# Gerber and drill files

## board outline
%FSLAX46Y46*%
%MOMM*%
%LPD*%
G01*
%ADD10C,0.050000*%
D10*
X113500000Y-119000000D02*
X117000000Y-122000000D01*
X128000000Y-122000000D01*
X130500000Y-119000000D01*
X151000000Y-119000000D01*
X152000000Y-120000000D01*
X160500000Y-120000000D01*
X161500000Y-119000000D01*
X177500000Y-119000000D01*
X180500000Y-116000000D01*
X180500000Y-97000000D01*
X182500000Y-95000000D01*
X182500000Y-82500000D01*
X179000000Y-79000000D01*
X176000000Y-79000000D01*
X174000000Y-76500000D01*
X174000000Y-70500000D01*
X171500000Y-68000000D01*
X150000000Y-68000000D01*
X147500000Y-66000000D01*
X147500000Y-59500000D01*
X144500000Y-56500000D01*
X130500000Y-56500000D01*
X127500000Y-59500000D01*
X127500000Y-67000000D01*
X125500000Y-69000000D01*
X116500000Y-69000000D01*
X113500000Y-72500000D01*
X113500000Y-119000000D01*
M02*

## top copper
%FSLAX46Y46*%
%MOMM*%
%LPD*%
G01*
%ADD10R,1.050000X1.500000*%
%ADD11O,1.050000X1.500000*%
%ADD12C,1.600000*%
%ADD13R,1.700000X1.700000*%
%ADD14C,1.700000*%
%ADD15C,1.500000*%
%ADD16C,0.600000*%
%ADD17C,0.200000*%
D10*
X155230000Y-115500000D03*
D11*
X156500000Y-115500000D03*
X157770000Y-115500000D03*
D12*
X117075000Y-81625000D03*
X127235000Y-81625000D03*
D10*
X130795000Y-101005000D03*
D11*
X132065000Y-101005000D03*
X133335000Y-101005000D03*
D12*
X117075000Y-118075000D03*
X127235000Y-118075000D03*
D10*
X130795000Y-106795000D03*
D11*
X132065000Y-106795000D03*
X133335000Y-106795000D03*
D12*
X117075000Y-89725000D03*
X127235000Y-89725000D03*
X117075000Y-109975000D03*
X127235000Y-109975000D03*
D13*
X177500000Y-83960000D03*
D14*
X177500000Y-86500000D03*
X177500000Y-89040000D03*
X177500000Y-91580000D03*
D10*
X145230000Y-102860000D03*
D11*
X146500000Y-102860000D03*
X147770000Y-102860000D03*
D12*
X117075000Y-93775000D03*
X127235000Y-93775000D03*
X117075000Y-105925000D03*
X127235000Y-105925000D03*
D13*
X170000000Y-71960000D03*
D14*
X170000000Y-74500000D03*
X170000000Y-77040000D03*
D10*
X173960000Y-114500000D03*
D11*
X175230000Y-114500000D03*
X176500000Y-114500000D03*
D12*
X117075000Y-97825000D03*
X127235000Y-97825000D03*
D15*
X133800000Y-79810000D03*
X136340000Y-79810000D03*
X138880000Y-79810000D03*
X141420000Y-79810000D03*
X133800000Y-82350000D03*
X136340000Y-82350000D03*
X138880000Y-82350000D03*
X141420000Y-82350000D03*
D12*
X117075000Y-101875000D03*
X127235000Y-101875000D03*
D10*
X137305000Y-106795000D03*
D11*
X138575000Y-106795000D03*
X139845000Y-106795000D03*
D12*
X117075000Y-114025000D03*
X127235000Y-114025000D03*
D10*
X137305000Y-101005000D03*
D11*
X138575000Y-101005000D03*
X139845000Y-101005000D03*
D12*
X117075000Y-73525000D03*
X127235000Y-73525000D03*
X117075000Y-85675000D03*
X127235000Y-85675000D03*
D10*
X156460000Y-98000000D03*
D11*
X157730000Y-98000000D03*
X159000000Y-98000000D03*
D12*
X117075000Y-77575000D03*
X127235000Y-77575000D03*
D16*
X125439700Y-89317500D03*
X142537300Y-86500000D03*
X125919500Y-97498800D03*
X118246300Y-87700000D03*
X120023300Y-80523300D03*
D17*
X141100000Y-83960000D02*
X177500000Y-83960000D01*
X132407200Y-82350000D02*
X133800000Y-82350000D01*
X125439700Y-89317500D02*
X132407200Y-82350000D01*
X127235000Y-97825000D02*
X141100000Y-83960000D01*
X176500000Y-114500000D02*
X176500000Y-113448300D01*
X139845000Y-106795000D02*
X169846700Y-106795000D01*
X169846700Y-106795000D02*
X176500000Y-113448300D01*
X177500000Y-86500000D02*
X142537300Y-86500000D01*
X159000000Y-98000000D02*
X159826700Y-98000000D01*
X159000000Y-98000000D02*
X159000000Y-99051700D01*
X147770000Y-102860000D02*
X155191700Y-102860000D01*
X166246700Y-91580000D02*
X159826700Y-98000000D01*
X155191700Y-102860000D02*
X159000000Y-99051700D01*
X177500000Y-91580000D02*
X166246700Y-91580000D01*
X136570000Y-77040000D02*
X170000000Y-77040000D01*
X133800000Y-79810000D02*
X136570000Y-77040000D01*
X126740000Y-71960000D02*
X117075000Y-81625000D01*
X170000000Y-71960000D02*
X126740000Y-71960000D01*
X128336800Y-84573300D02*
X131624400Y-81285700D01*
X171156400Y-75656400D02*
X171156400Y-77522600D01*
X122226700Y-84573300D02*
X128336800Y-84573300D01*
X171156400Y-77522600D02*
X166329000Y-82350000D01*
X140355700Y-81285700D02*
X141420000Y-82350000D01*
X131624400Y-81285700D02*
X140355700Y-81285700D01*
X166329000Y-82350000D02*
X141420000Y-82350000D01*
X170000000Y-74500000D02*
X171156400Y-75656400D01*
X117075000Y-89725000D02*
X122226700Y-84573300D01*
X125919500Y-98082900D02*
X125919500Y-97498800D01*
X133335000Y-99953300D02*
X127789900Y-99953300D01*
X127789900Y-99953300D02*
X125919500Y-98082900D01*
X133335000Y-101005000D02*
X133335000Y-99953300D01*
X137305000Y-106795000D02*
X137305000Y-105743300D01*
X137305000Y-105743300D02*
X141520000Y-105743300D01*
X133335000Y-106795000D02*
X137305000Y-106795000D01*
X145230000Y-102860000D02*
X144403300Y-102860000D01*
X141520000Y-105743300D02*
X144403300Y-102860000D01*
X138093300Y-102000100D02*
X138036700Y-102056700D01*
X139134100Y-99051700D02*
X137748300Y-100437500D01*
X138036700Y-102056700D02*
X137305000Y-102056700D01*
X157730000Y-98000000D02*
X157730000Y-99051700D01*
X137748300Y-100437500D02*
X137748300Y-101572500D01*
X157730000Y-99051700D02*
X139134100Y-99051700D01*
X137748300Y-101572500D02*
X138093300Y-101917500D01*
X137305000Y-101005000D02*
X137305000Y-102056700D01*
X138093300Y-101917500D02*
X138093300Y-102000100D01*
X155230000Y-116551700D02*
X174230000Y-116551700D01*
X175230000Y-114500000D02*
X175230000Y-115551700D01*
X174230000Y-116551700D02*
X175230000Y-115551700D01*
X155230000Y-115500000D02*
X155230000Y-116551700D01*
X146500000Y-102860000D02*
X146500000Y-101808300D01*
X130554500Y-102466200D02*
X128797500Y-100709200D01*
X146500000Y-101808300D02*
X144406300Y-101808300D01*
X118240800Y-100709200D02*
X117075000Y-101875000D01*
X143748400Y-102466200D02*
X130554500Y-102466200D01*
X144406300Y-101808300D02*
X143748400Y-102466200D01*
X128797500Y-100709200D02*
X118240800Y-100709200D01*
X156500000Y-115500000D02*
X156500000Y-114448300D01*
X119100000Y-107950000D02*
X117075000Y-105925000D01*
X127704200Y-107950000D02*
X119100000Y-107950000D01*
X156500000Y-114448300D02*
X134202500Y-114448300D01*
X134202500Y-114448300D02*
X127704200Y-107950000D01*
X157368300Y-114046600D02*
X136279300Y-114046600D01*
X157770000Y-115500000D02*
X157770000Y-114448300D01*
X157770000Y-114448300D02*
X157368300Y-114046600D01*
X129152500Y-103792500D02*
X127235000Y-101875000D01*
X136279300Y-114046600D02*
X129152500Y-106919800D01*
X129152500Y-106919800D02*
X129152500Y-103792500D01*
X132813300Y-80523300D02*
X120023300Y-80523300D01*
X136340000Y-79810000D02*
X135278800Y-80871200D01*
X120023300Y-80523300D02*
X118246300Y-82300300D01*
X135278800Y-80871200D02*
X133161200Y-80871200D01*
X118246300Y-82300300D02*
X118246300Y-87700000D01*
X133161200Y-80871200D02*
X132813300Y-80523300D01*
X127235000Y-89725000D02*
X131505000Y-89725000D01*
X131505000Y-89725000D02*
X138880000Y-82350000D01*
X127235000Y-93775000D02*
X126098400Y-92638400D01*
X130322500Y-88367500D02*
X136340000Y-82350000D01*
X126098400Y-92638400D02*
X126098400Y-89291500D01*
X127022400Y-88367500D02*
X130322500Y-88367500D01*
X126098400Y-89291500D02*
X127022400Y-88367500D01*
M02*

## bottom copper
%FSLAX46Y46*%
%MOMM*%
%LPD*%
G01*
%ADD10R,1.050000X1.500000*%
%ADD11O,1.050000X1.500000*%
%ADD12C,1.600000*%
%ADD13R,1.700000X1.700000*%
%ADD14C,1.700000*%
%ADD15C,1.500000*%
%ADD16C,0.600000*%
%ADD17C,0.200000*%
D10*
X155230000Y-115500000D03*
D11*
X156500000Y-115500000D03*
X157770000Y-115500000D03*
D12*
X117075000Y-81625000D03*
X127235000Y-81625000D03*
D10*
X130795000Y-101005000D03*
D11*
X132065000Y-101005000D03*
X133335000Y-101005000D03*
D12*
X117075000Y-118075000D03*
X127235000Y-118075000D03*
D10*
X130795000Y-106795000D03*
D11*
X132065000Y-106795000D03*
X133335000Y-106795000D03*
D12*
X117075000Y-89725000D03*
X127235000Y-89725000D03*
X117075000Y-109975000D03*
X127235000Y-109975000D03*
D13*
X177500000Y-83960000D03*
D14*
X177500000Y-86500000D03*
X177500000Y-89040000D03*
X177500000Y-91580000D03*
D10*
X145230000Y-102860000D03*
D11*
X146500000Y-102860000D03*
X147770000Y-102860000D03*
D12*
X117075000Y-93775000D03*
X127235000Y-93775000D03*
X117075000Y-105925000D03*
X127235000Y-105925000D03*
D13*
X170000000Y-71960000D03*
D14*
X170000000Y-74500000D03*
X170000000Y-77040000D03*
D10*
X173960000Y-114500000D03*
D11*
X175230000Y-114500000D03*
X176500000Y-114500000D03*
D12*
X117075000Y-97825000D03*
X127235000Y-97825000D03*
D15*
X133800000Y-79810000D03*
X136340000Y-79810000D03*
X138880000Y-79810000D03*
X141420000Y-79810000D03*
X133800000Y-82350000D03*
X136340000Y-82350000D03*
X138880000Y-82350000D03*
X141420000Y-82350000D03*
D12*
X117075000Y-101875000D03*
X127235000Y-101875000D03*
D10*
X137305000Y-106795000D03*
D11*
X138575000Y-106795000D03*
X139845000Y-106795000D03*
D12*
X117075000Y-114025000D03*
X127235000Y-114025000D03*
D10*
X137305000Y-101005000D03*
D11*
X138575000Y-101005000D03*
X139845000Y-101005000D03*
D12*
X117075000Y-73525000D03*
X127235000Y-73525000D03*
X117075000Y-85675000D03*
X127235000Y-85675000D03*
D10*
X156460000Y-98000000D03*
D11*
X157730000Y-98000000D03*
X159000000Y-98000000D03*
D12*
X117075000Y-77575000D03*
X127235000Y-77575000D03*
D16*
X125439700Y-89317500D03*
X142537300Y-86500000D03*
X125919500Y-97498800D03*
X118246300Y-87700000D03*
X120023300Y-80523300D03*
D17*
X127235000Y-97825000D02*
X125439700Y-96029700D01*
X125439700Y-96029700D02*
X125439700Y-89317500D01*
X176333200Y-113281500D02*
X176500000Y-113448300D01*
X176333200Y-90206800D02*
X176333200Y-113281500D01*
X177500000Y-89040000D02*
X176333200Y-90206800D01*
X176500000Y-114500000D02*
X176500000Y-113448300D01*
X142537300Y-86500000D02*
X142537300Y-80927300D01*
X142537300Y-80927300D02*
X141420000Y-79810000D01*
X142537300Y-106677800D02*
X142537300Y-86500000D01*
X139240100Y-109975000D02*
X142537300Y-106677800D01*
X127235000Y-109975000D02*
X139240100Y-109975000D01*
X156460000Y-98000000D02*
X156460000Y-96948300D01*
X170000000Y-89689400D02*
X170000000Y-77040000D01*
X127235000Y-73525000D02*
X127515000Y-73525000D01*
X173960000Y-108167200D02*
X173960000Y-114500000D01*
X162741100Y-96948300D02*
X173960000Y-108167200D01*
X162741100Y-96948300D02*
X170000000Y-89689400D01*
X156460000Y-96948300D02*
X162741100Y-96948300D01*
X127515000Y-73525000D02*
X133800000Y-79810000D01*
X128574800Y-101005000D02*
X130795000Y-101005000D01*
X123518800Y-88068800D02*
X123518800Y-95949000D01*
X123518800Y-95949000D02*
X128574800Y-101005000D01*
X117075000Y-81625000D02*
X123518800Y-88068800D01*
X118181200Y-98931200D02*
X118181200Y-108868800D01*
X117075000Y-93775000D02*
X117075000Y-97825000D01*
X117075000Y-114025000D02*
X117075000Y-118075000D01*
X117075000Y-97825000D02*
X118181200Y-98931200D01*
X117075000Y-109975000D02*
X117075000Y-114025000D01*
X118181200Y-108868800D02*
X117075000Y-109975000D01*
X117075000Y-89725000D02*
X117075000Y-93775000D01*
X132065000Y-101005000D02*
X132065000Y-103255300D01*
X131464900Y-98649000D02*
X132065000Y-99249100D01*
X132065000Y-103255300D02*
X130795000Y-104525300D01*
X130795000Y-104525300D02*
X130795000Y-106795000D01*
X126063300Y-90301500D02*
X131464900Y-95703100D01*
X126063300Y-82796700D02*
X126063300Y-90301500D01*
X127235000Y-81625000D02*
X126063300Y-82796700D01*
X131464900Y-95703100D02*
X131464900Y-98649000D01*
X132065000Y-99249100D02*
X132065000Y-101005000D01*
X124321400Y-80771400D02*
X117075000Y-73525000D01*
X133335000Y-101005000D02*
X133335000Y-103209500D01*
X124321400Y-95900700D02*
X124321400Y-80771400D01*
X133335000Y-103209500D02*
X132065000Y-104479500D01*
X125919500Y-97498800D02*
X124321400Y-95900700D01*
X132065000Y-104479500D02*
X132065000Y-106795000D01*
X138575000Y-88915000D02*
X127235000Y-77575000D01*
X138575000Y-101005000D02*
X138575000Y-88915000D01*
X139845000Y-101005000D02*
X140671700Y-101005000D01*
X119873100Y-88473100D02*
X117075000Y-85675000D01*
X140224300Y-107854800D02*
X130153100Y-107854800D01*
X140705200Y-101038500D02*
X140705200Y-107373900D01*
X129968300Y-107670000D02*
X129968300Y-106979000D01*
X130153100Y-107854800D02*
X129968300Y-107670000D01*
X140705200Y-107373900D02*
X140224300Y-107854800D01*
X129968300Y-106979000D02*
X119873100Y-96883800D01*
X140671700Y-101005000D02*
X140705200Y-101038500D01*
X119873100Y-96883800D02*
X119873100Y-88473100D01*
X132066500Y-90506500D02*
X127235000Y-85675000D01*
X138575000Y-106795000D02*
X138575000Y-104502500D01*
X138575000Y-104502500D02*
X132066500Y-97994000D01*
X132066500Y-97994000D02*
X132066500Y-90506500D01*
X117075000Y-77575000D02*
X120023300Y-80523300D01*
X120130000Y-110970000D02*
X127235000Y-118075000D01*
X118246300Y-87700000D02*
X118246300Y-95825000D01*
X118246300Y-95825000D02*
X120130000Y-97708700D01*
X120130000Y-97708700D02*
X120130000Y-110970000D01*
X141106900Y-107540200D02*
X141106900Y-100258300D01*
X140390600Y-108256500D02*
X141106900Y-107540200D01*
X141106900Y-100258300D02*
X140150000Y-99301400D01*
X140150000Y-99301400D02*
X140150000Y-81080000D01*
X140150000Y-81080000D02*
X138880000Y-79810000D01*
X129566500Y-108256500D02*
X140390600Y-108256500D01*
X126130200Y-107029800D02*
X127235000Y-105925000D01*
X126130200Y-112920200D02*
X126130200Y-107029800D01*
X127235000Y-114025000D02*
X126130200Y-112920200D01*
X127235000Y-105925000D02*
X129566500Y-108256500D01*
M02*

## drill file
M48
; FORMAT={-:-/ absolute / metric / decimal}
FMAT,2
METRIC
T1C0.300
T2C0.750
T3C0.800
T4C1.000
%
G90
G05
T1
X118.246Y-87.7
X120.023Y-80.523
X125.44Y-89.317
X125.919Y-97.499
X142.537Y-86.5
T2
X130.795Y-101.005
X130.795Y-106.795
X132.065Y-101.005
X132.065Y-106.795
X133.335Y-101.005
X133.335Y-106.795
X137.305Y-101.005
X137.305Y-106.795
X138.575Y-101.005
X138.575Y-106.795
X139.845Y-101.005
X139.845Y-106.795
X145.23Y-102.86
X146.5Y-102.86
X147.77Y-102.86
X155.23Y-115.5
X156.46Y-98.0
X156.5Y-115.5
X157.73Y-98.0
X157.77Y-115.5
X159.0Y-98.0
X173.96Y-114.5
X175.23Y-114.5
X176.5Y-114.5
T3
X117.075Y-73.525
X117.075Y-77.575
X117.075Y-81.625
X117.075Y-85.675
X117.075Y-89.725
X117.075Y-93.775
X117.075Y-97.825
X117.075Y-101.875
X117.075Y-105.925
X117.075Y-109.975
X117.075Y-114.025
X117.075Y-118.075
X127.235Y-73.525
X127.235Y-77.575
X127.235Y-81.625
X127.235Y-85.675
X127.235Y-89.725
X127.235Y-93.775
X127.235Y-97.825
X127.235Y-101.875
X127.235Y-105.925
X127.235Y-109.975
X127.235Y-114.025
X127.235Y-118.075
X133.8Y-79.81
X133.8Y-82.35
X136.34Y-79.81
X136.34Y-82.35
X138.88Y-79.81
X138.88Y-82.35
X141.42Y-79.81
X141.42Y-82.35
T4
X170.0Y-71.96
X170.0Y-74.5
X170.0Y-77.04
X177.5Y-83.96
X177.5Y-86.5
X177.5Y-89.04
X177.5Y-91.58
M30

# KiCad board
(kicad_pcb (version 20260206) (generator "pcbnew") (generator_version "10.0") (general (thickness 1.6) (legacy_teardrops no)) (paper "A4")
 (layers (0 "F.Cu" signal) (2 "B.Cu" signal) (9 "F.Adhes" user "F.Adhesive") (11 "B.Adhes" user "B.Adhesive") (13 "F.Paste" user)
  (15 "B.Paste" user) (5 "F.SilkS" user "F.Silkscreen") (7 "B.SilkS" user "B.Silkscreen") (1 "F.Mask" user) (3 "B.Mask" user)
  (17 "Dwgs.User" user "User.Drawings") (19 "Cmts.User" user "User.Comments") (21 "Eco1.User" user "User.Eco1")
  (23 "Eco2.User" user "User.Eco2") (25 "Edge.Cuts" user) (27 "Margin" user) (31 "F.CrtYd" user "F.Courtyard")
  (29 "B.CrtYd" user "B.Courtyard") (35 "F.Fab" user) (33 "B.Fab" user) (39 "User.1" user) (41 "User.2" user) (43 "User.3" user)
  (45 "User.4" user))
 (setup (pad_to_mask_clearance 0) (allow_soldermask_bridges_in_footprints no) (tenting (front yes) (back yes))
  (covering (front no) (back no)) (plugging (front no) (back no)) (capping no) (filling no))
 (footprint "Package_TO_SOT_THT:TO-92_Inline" (layer "F.Cu") (at 155.23 115.5)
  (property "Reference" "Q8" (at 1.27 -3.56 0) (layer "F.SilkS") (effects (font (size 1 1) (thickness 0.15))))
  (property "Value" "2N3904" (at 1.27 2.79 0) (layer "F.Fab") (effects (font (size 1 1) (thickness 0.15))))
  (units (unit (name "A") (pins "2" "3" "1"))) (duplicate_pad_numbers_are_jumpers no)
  (pad "1" thru_hole rect (at 0 0) (size 1.05 1.5) (drill 0.75) (layers "*.Cu" "*.Mask") (remove_unused_layers no) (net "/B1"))
  (pad "2" thru_hole oval (at 1.27 0) (size 1.05 1.5) (drill 0.75) (layers "*.Cu" "*.Mask") (remove_unused_layers no) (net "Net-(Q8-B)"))
  (pad "3" thru_hole oval (at 2.54 0) (size 1.05 1.5) (drill 0.75) (layers "*.Cu" "*.Mask") (remove_unused_layers no) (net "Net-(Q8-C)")))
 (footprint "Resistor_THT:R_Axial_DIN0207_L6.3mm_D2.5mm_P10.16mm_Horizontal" (layer "F.Cu") (at 117.075 81.625)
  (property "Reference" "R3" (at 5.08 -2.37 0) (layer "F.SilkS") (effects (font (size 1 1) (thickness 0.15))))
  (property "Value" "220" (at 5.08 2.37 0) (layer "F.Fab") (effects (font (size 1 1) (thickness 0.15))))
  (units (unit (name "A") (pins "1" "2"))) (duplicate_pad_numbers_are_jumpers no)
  (pad "1" thru_hole circle (at 0 0) (size 1.6 1.6) (drill 0.8) (layers "*.Cu" "*.Mask") (remove_unused_layers no) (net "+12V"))
  (pad "2" thru_hole circle (at 10.16 0) (size 1.6 1.6) (drill 0.8) (layers "*.Cu" "*.Mask") (remove_unused_layers no) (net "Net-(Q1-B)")))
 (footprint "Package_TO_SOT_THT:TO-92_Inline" (layer "F.Cu") (at 130.795 101.005)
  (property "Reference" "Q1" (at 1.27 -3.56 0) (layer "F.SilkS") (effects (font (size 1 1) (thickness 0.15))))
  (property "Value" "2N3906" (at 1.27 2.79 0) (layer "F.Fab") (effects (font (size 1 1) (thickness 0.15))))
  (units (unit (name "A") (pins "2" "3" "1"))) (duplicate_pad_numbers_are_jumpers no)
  (pad "1" thru_hole rect (at 0 0) (size 1.05 1.5) (drill 0.75) (layers "*.Cu" "*.Mask") (remove_unused_layers no) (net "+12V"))
  (pad "2" thru_hole oval (at 1.27 0) (size 1.05 1.5) (drill 0.75) (layers "*.Cu" "*.Mask") (remove_unused_layers no) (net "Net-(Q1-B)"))
  (pad "3" thru_hole oval (at 2.54 0) (size 1.05 1.5) (drill 0.75) (layers "*.Cu" "*.Mask") (remove_unused_layers no) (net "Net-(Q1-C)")))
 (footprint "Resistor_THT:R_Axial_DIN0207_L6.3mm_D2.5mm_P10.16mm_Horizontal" (layer "F.Cu") (at 117.075 118.075)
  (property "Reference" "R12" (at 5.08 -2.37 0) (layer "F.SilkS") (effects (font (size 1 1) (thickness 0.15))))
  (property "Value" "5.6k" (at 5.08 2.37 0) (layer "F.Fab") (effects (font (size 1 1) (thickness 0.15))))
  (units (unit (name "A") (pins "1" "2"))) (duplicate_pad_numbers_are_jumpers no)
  (pad "1" thru_hole circle (at 0 0) (size 1.6 1.6) (drill 0.8) (layers "*.Cu" "*.Mask") (remove_unused_layers no) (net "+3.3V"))
  (pad "2" thru_hole circle (at 10.16 0) (size 1.6 1.6) (drill 0.8) (layers "*.Cu" "*.Mask") (remove_unused_layers no) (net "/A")))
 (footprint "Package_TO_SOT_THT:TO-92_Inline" (layer "F.Cu") (at 130.795 106.795)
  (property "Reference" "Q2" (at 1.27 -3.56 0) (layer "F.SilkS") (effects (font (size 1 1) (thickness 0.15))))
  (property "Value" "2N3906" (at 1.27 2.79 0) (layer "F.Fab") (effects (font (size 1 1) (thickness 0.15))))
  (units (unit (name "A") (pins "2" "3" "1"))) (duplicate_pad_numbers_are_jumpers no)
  (pad "1" thru_hole rect (at 0 0) (size 1.05 1.5) (drill 0.75) (layers "*.Cu" "*.Mask") (remove_unused_layers no) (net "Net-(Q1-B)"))
  (pad "2" thru_hole oval (at 1.27 0) (size 1.05 1.5) (drill 0.75) (layers "*.Cu" "*.Mask") (remove_unused_layers no) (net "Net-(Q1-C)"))
  (pad "3" thru_hole oval (at 2.54 0) (size 1.05 1.5) (drill 0.75) (layers "*.Cu" "*.Mask") (remove_unused_layers no) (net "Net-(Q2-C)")))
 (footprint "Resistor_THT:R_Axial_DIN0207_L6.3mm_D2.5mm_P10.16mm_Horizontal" (layer "F.Cu") (at 117.075 89.725)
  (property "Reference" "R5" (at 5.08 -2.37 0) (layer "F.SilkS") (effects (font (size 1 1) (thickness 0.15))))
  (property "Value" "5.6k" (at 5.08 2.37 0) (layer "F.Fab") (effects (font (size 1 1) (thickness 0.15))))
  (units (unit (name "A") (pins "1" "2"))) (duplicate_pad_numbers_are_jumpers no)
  (pad "1" thru_hole circle (at 0 0) (size 1.6 1.6) (drill 0.8) (layers "*.Cu" "*.Mask") (remove_unused_layers no) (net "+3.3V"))
  (pad "2" thru_hole circle (at 10.16 0) (size 1.6 1.6) (drill 0.8) (layers "*.Cu" "*.Mask") (remove_unused_layers no)
   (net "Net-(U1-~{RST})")))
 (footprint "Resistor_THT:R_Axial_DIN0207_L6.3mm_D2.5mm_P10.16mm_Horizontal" (layer "F.Cu") (at 117.075 109.975)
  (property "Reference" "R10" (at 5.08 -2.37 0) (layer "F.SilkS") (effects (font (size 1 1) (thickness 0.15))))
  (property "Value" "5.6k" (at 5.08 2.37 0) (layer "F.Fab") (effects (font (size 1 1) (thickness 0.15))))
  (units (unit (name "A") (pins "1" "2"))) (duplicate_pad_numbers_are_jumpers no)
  (pad "1" thru_hole circle (at 0 0) (size 1.6 1.6) (drill 0.8) (layers "*.Cu" "*.Mask") (remove_unused_layers no) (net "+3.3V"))
  (pad "2" thru_hole circle (at 10.16 0) (size 1.6 1.6) (drill 0.8) (layers "*.Cu" "*.Mask") (remove_unused_layers no) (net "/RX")))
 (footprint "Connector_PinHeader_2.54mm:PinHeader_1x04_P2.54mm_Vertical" (layer "F.Cu") (at 177.5 83.96)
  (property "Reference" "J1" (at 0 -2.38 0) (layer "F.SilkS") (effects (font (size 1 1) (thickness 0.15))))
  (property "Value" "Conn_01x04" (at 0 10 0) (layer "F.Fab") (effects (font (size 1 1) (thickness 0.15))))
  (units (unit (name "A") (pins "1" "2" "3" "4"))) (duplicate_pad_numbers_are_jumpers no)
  (pad "1" thru_hole rect (at 0 0) (size 1.7 1.7) (drill 1) (layers "*.Cu" "*.Mask") (remove_unused_layers no) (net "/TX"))
  (pad "2" thru_hole circle (at 0 2.54) (size 1.7 1.7) (drill 1) (layers "*.Cu" "*.Mask") (remove_unused_layers no) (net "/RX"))
  (pad "3" thru_hole circle (at 0 5.08) (size 1.7 1.7) (drill 1) (layers "*.Cu" "*.Mask") (remove_unused_layers no) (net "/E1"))
  (pad "4" thru_hole circle (at 0 7.62) (size 1.7 1.7) (drill 1) (layers "*.Cu" "*.Mask") (remove_unused_layers no) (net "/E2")))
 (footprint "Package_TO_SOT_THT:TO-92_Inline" (layer "F.Cu") (at 145.23 102.86)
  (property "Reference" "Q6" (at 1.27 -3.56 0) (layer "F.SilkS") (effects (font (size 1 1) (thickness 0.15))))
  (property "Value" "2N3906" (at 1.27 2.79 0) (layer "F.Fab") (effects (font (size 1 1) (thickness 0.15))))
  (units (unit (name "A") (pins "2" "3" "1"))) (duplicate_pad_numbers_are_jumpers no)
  (pad "1" thru_hole rect (at 0 0) (size 1.05 1.5) (drill 0.75) (layers "*.Cu" "*.Mask") (remove_unused_layers no) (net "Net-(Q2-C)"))
  (pad "2" thru_hole oval (at 1.27 0) (size 1.05 1.5) (drill 0.75) (layers "*.Cu" "*.Mask") (remove_unused_layers no) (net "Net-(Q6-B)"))
  (pad "3" thru_hole oval (at 2.54 0) (size 1.05 1.5) (drill 0.75) (layers "*.Cu" "*.Mask") (remove_unused_layers no) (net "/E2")))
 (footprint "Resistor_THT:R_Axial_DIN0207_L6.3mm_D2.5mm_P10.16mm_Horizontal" (layer "F.Cu") (at 117.075 93.775)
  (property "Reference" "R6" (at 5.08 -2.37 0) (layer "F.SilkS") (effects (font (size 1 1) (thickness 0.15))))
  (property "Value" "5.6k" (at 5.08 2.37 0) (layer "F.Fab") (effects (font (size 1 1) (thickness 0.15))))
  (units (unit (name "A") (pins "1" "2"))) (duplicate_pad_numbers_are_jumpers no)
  (pad "1" thru_hole circle (at 0 0) (size 1.6 1.6) (drill 0.8) (layers "*.Cu" "*.Mask") (remove_unused_layers no) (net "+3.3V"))
  (pad "2" thru_hole circle (at 10.16 0) (size 1.6 1.6) (drill 0.8) (layers "*.Cu" "*.Mask") (remove_unused_layers no) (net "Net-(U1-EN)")))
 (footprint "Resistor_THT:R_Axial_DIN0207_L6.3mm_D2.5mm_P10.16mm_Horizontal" (layer "F.Cu") (at 117.075 105.925)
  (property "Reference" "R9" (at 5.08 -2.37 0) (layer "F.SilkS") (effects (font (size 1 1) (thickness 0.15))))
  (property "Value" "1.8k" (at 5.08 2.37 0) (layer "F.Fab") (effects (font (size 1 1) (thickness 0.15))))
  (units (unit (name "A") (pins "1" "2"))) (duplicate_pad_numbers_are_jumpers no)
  (pad "1" thru_hole circle (at 0 0) (size 1.6 1.6) (drill 0.8) (layers "*.Cu" "*.Mask") (remove_unused_layers no) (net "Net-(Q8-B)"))
  (pad "2" thru_hole circle (at 10.16 0) (size 1.6 1.6) (drill 0.8) (layers "*.Cu" "*.Mask") (remove_unused_layers no) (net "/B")))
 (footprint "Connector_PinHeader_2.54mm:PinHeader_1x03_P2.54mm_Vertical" (layer "F.Cu") (at 170 71.96)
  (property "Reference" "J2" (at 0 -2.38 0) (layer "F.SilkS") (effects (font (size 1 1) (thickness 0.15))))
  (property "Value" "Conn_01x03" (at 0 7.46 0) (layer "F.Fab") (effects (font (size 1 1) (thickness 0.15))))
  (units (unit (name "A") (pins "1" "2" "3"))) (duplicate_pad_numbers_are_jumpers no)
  (pad "1" thru_hole rect (at 0 0) (size 1.7 1.7) (drill 1) (layers "*.Cu" "*.Mask") (remove_unused_layers no) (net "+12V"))
  (pad "2" thru_hole circle (at 0 2.54) (size 1.7 1.7) (drill 1) (layers "*.Cu" "*.Mask") (remove_unused_layers no) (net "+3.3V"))
  (pad "3" thru_hole circle (at 0 5.08) (size 1.7 1.7) (drill 1) (layers "*.Cu" "*.Mask") (remove_unused_layers no) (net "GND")))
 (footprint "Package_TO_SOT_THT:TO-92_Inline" (layer "F.Cu") (at 173.96 114.5)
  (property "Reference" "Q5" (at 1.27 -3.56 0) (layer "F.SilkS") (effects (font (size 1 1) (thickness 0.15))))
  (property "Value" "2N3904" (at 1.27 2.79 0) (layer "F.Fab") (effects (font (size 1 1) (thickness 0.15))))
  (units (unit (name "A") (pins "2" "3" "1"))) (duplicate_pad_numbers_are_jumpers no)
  (pad "1" thru_hole rect (at 0 0) (size 1.05 1.5) (drill 0.75) (layers "*.Cu" "*.Mask") (remove_unused_layers no) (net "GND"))
  (pad "2" thru_hole oval (at 1.27 0) (size 1.05 1.5) (drill 0.75) (layers "*.Cu" "*.Mask") (remove_unused_layers no) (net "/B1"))
  (pad "3" thru_hole oval (at 2.54 0) (size 1.05 1.5) (drill 0.75) (layers "*.Cu" "*.Mask") (remove_unused_layers no) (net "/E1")))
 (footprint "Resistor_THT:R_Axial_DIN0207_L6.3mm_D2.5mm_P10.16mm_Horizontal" (layer "F.Cu") (at 117.075 97.825)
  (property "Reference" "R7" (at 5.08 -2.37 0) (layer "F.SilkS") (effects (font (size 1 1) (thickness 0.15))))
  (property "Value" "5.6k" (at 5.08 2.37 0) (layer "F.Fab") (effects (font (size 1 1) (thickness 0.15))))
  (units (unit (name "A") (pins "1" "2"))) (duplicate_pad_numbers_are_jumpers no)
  (pad "1" thru_hole circle (at 0 0) (size 1.6 1.6) (drill 0.8) (layers "*.Cu" "*.Mask") (remove_unused_layers no) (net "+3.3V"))
  (pad "2" thru_hole circle (at 10.16 0) (size 1.6 1.6) (drill 0.8) (layers "*.Cu" "*.Mask") (remove_unused_layers no) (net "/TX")))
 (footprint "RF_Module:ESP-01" (layer "F.Cu") (at 133.8 79.81)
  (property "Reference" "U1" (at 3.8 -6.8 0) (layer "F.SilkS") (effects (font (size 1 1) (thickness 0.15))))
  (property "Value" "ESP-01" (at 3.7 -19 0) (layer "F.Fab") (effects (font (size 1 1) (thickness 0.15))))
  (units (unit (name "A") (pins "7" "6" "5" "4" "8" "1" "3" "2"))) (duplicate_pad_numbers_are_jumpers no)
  (pad "1" thru_hole circle (at 0 0) (size 1.5 1.5) (drill 0.8) (layers "*.Cu" "*.Mask") (remove_unused_layers no) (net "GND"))
  (pad "2" thru_hole circle (at 2.54 0) (size 1.5 1.5) (drill 0.8) (layers "*.Cu" "*.Mask") (remove_unused_layers no) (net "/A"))
  (pad "3" thru_hole circle (at 5.08 0) (size 1.5 1.5) (drill 0.8) (layers "*.Cu" "*.Mask") (remove_unused_layers no) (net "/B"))
  (pad "4" thru_hole circle (at 7.62 0) (size 1.5 1.5) (drill 0.8) (layers "*.Cu" "*.Mask") (remove_unused_layers no) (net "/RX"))
  (pad "5" thru_hole circle (at 0 2.54) (size 1.5 1.5) (drill 0.8) (layers "*.Cu" "*.Mask") (remove_unused_layers no) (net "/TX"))
  (pad "6" thru_hole circle (at 2.54 2.54) (size 1.5 1.5) (drill 0.8) (layers "*.Cu" "*.Mask") (remove_unused_layers no) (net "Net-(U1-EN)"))
  (pad "7" thru_hole circle (at 5.08 2.54) (size 1.5 1.5) (drill 0.8) (layers "*.Cu" "*.Mask") (remove_unused_layers no)
   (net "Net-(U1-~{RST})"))
  (pad "8" thru_hole circle (at 7.62 2.54) (size 1.5 1.5) (drill 0.8) (layers "*.Cu" "*.Mask") (remove_unused_layers no) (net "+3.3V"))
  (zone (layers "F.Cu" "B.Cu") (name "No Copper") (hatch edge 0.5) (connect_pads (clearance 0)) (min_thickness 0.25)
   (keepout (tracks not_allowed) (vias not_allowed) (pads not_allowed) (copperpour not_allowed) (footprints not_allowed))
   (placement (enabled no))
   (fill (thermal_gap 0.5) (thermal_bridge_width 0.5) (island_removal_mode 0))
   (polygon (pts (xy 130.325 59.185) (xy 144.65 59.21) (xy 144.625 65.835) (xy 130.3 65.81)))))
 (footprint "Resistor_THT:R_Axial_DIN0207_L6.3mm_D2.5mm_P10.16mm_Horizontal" (layer "F.Cu") (at 117.075 101.875)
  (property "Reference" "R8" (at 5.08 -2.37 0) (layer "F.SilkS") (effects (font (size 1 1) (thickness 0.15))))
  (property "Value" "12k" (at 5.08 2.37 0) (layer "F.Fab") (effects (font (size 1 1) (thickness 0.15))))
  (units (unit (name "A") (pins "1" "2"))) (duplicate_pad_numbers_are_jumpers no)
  (pad "1" thru_hole circle (at 0 0) (size 1.6 1.6) (drill 0.8) (layers "*.Cu" "*.Mask") (remove_unused_layers no) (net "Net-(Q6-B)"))
  (pad "2" thru_hole circle (at 10.16 0) (size 1.6 1.6) (drill 0.8) (layers "*.Cu" "*.Mask") (remove_unused_layers no) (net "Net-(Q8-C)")))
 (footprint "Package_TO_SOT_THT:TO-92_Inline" (layer "F.Cu") (at 137.305 106.795)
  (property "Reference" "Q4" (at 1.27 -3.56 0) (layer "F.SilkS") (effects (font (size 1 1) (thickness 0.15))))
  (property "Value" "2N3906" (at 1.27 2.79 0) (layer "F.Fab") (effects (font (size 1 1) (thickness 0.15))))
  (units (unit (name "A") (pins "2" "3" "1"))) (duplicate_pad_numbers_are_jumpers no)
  (pad "1" thru_hole rect (at 0 0) (size 1.05 1.5) (drill 0.75) (layers "*.Cu" "*.Mask") (remove_unused_layers no) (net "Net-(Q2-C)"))
  (pad "2" thru_hole oval (at 1.27 0) (size 1.05 1.5) (drill 0.75) (layers "*.Cu" "*.Mask") (remove_unused_layers no) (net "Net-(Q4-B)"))
  (pad "3" thru_hole oval (at 2.54 0) (size 1.05 1.5) (drill 0.75) (layers "*.Cu" "*.Mask") (remove_unused_layers no) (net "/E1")))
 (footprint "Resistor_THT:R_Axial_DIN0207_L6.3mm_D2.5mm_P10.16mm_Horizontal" (layer "F.Cu") (at 117.075 114.025)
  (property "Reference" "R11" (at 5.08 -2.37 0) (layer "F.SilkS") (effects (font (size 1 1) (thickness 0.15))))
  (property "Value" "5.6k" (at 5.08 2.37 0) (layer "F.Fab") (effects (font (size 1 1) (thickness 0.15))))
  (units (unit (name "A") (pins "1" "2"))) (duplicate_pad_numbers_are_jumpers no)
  (pad "1" thru_hole circle (at 0 0) (size 1.6 1.6) (drill 0.8) (layers "*.Cu" "*.Mask") (remove_unused_layers no) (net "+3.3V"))
  (pad "2" thru_hole circle (at 10.16 0) (size 1.6 1.6) (drill 0.8) (layers "*.Cu" "*.Mask") (remove_unused_layers no) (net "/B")))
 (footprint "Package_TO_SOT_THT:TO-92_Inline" (layer "F.Cu") (at 137.305 101.005)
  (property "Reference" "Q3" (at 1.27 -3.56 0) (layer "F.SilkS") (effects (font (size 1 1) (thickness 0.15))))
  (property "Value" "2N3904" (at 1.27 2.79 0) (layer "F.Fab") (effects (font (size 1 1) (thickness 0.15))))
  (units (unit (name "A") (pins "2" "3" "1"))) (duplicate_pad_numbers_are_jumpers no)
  (pad "1" thru_hole rect (at 0 0) (size 1.05 1.5) (drill 0.75) (layers "*.Cu" "*.Mask") (remove_unused_layers no) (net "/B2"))
  (pad "2" thru_hole oval (at 1.27 0) (size 1.05 1.5) (drill 0.75) (layers "*.Cu" "*.Mask") (remove_unused_layers no) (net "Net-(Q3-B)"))
  (pad "3" thru_hole oval (at 2.54 0) (size 1.05 1.5) (drill 0.75) (layers "*.Cu" "*.Mask") (remove_unused_layers no) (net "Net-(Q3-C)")))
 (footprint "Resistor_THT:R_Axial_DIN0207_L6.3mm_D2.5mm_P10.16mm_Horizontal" (layer "F.Cu") (at 117.075 73.525)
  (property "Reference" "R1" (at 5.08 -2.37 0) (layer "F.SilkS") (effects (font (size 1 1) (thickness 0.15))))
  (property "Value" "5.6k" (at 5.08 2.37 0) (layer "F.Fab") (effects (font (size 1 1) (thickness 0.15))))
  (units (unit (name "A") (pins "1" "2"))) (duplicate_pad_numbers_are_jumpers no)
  (pad "1" thru_hole circle (at 0 0) (size 1.6 1.6) (drill 0.8) (layers "*.Cu" "*.Mask") (remove_unused_layers no) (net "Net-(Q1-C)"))
  (pad "2" thru_hole circle (at 10.16 0) (size 1.6 1.6) (drill 0.8) (layers "*.Cu" "*.Mask") (remove_unused_layers no) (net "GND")))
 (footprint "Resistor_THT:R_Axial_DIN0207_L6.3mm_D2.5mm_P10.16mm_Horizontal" (layer "F.Cu") (at 117.075 85.675)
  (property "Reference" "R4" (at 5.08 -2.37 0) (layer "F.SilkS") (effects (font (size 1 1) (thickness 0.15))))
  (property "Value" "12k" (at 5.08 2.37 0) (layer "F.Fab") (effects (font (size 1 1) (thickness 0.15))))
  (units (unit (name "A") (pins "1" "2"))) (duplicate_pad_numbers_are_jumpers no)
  (pad "1" thru_hole circle (at 0 0) (size 1.6 1.6) (drill 0.8) (layers "*.Cu" "*.Mask") (remove_unused_layers no) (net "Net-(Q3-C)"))
  (pad "2" thru_hole circle (at 10.16 0) (size 1.6 1.6) (drill 0.8) (layers "*.Cu" "*.Mask") (remove_unused_layers no) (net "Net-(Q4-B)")))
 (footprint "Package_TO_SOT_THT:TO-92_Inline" (layer "F.Cu") (at 156.46 98)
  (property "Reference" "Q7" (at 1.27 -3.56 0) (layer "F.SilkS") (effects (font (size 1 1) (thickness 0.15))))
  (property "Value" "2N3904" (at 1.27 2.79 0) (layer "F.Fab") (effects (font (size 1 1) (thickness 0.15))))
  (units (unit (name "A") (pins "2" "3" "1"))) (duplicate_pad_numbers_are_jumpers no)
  (pad "1" thru_hole rect (at 0 0) (size 1.05 1.5) (drill 0.75) (layers "*.Cu" "*.Mask") (remove_unused_layers no) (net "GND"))
  (pad "2" thru_hole oval (at 1.27 0) (size 1.05 1.5) (drill 0.75) (layers "*.Cu" "*.Mask") (remove_unused_layers no) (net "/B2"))
  (pad "3" thru_hole oval (at 2.54 0) (size 1.05 1.5) (drill 0.75) (layers "*.Cu" "*.Mask") (remove_unused_layers no) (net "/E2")))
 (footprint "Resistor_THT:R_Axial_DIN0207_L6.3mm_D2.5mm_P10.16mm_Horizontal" (layer "F.Cu") (at 117.075 77.575)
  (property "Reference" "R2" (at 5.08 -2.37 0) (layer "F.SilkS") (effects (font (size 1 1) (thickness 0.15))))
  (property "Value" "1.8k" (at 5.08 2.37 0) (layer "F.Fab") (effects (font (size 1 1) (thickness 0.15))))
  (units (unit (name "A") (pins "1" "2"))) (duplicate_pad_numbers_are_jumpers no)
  (pad "1" thru_hole circle (at 0 0) (size 1.6 1.6) (drill 0.8) (layers "*.Cu" "*.Mask") (remove_unused_layers no) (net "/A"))
  (pad "2" thru_hole circle (at 10.16 0) (size 1.6 1.6) (drill 0.8) (layers "*.Cu" "*.Mask") (remove_unused_layers no) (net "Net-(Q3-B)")))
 (gr_poly
  (pts (xy 113.5 119) (xy 117 122) (xy 128 122) (xy 130.5 119) (xy 151 119) (xy 152 120) (xy 160.5 120) (xy 161.5 119) (xy 177.5 119)
   (xy 180.5 116) (xy 180.5 97) (xy 182.5 95) (xy 182.5 82.5) (xy 179 79) (xy 176 79) (xy 174 76.5) (xy 174 70.5) (xy 171.5 68) (xy 150 68)
   (xy 147.5 66) (xy 147.5 59.5) (xy 144.5 56.5) (xy 130.5 56.5) (xy 127.5 59.5) (xy 127.5 67) (xy 125.5 69) (xy 116.5 69) (xy 113.5 72.5))
  (stroke (width 0.05) (type solid)) (fill no) (layer "Edge.Cuts"))
 (segment (start 141.1 83.96) (end 177.5 83.96) (width 0.2) (layer "F.Cu") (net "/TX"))
 (segment (start 132.4072 82.35) (end 133.8 82.35) (width 0.2) (layer "F.Cu") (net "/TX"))
 (segment (start 125.4397 89.3175) (end 132.4072 82.35) (width 0.2) (layer "F.Cu") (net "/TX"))
 (segment (start 127.235 97.825) (end 141.1 83.96) (width 0.2) (layer "F.Cu") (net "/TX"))
 (via (at 125.4397 89.3175) (size 0.6) (drill 0.3) (layers "F.Cu" "B.Cu") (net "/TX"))
 (segment (start 127.235 97.825) (end 125.4397 96.0297) (width 0.2) (layer "B.Cu") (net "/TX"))
 (segment (start 125.4397 96.0297) (end 125.4397 89.3175) (width 0.2) (layer "B.Cu") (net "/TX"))
 (segment (start 176.5 114.5) (end 176.5 113.4483) (width 0.2) (layer "F.Cu") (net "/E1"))
 (segment (start 139.845 106.795) (end 169.8467 106.795) (width 0.2) (layer "F.Cu") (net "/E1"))
 (segment (start 169.8467 106.795) (end 176.5 113.4483) (width 0.2) (layer "F.Cu") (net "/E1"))
 (segment (start 176.3332 113.2815) (end 176.5 113.4483) (width 0.2) (layer "B.Cu") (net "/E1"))
 (segment (start 176.3332 90.2068) (end 176.3332 113.2815) (width 0.2) (layer "B.Cu") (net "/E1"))
 (segment (start 177.5 89.04) (end 176.3332 90.2068) (width 0.2) (layer "B.Cu") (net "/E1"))
 (segment (start 176.5 114.5) (end 176.5 113.4483) (width 0.2) (layer "B.Cu") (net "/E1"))
 (segment (start 177.5 86.5) (end 142.5373 86.5) (width 0.2) (layer "F.Cu") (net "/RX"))
 (via (at 142.5373 86.5) (size 0.6) (drill 0.3) (layers "F.Cu" "B.Cu") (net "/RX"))
 (segment (start 142.5373 86.5) (end 142.5373 80.9273) (width 0.2) (layer "B.Cu") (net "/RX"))
 (segment (start 142.5373 80.9273) (end 141.42 79.81) (width 0.2) (layer "B.Cu") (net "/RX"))
 (segment (start 142.5373 106.6778) (end 142.5373 86.5) (width 0.2) (layer "B.Cu") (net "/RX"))
 (segment (start 139.2401 109.975) (end 142.5373 106.6778) (width 0.2) (layer "B.Cu") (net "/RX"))
 (segment (start 127.235 109.975) (end 139.2401 109.975) (width 0.2) (layer "B.Cu") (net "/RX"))
 (segment (start 159 98) (end 159.8267 98) (width 0.2) (layer "F.Cu") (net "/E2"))
 (segment (start 159 98) (end 159 99.0517) (width 0.2) (layer "F.Cu") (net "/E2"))
 (segment (start 147.77 102.86) (end 155.1917 102.86) (width 0.2) (layer "F.Cu") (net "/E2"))
 (segment (start 166.2467 91.58) (end 159.8267 98) (width 0.2) (layer "F.Cu") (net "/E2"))
 (segment (start 155.1917 102.86) (end 159 99.0517) (width 0.2) (layer "F.Cu") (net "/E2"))
 (segment (start 177.5 91.58) (end 166.2467 91.58) (width 0.2) (layer "F.Cu") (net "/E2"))
 (segment (start 136.57 77.04) (end 170 77.04) (width 0.2) (layer "F.Cu") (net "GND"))
 (segment (start 133.8 79.81) (end 136.57 77.04) (width 0.2) (layer "F.Cu") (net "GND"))
 (segment (start 156.46 98) (end 156.46 96.9483) (width 0.2) (layer "B.Cu") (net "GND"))
 (segment (start 170 89.6894) (end 170 77.04) (width 0.2) (layer "B.Cu") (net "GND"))
 (segment (start 127.235 73.525) (end 127.515 73.525) (width 0.2) (layer "B.Cu") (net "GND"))
 (segment (start 173.96 108.1672) (end 173.96 114.5) (width 0.2) (layer "B.Cu") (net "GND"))
 (segment (start 162.7411 96.9483) (end 173.96 108.1672) (width 0.2) (layer "B.Cu") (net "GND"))
 (segment (start 162.7411 96.9483) (end 170 89.6894) (width 0.2) (layer "B.Cu") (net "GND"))
 (segment (start 156.46 96.9483) (end 162.7411 96.9483) (width 0.2) (layer "B.Cu") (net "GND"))
 (segment (start 127.515 73.525) (end 133.8 79.81) (width 0.2) (layer "B.Cu") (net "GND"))
 (segment (start 126.74 71.96) (end 117.075 81.625) (width 0.2) (layer "F.Cu") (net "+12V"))
 (segment (start 170 71.96) (end 126.74 71.96) (width 0.2) (layer "F.Cu") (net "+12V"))
 (segment (start 128.5748 101.005) (end 130.795 101.005) (width 0.2) (layer "B.Cu") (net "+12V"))
 (segment (start 123.5188 88.0688) (end 123.5188 95.949) (width 0.2) (layer "B.Cu") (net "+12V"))
 (segment (start 123.5188 95.949) (end 128.5748 101.005) (width 0.2) (layer "B.Cu") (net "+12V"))
 (segment (start 117.075 81.625) (end 123.5188 88.0688) (width 0.2) (layer "B.Cu") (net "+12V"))
 (segment (start 128.3368 84.5733) (end 131.6244 81.2857) (width 0.2) (layer "F.Cu") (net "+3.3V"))
 (segment (start 171.1564 75.6564) (end 171.1564 77.5226) (width 0.2) (layer "F.Cu") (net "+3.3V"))
 (segment (start 122.2267 84.5733) (end 128.3368 84.5733) (width 0.2) (layer "F.Cu") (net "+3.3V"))
 (segment (start 171.1564 77.5226) (end 166.329 82.35) (width 0.2) (layer "F.Cu") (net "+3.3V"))
 (segment (start 140.3557 81.2857) (end 141.42 82.35) (width 0.2) (layer "F.Cu") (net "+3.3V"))
 (segment (start 131.6244 81.2857) (end 140.3557 81.2857) (width 0.2) (layer "F.Cu") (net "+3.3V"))
 (segment (start 166.329 82.35) (end 141.42 82.35) (width 0.2) (layer "F.Cu") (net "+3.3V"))
 (segment (start 170 74.5) (end 171.1564 75.6564) (width 0.2) (layer "F.Cu") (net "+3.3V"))
 (segment (start 117.075 89.725) (end 122.2267 84.5733) (width 0.2) (layer "F.Cu") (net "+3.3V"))
 (segment (start 118.1812 98.9312) (end 118.1812 108.8688) (width 0.2) (layer "B.Cu") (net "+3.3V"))
 (segment (start 117.075 93.775) (end 117.075 97.825) (width 0.2) (layer "B.Cu") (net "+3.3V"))
 (segment (start 117.075 114.025) (end 117.075 118.075) (width 0.2) (layer "B.Cu") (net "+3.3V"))
 (segment (start 117.075 97.825) (end 118.1812 98.9312) (width 0.2) (layer "B.Cu") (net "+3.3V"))
 (segment (start 117.075 109.975) (end 117.075 114.025) (width 0.2) (layer "B.Cu") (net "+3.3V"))
 (segment (start 118.1812 108.8688) (end 117.075 109.975) (width 0.2) (layer "B.Cu") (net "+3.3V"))
 (segment (start 117.075 89.725) (end 117.075 93.775) (width 0.2) (layer "B.Cu") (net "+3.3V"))
 (segment (start 132.065 101.005) (end 132.065 103.2553) (width 0.2) (layer "B.Cu") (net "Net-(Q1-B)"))
 (segment (start 131.4649 98.649) (end 132.065 99.2491) (width 0.2) (layer "B.Cu") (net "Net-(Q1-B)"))
 (segment (start 132.065 103.2553) (end 130.795 104.5253) (width 0.2) (layer "B.Cu") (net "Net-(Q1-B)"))
 (segment (start 130.795 104.5253) (end 130.795 106.795) (width 0.2) (layer "B.Cu") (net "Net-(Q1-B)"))
 (segment (start 126.0633 90.3015) (end 131.4649 95.7031) (width 0.2) (layer "B.Cu") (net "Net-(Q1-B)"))
 (segment (start 126.0633 82.7967) (end 126.0633 90.3015) (width 0.2) (layer "B.Cu") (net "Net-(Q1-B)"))
 (segment (start 127.235 81.625) (end 126.0633 82.7967) (width 0.2) (layer "B.Cu") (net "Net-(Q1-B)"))
 (segment (start 131.4649 95.7031) (end 131.4649 98.649) (width 0.2) (layer "B.Cu") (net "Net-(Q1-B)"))
 (segment (start 132.065 99.2491) (end 132.065 101.005) (width 0.2) (layer "B.Cu") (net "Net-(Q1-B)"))
 (segment (start 125.9195 98.0829) (end 125.9195 97.4988) (width 0.2) (layer "F.Cu") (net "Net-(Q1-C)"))
 (segment (start 133.335 99.9533) (end 127.7899 99.9533) (width 0.2) (layer "F.Cu") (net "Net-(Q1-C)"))
 (segment (start 127.7899 99.9533) (end 125.9195 98.0829) (width 0.2) (layer "F.Cu") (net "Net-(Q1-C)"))
 (segment (start 133.335 101.005) (end 133.335 99.9533) (width 0.2) (layer "F.Cu") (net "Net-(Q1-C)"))
 (via (at 125.9195 97.4988) (size 0.6) (drill 0.3) (layers "F.Cu" "B.Cu") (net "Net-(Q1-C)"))
 (segment (start 124.3214 80.7714) (end 117.075 73.525) (width 0.2) (layer "B.Cu") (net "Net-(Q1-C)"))
 (segment (start 133.335 101.005) (end 133.335 103.2095) (width 0.2) (layer "B.Cu") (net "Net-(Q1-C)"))
 (segment (start 124.3214 95.9007) (end 124.3214 80.7714) (width 0.2) (layer "B.Cu") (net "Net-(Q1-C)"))
 (segment (start 133.335 103.2095) (end 132.065 104.4795) (width 0.2) (layer "B.Cu") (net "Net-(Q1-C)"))
 (segment (start 125.9195 97.4988) (end 124.3214 95.9007) (width 0.2) (layer "B.Cu") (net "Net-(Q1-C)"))
 (segment (start 132.065 104.4795) (end 132.065 106.795) (width 0.2) (layer "B.Cu") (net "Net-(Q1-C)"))
 (segment (start 137.305 106.795) (end 137.305 105.7433) (width 0.2) (layer "F.Cu") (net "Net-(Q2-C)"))
 (segment (start 137.305 105.7433) (end 141.52 105.7433) (width 0.2) (layer "F.Cu") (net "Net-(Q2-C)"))
 (segment (start 133.335 106.795) (end 137.305 106.795) (width 0.2) (layer "F.Cu") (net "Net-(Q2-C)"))
 (segment (start 145.23 102.86) (end 144.4033 102.86) (width 0.2) (layer "F.Cu") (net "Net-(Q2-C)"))
 (segment (start 141.52 105.7433) (end 144.4033 102.86) (width 0.2) (layer "F.Cu") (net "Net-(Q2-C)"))
 (segment (start 138.575 88.915) (end 127.235 77.575) (width 0.2) (layer "B.Cu") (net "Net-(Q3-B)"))
 (segment (start 138.575 101.005) (end 138.575 88.915) (width 0.2) (layer "B.Cu") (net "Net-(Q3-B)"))
 (segment (start 138.0933 102.0001) (end 138.0367 102.0567) (width 0.2) (layer "F.Cu") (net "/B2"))
 (segment (start 139.1341 99.0517) (end 137.7483 100.4375) (width 0.2) (layer "F.Cu") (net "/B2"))
 (segment (start 138.0367 102.0567) (end 137.305 102.0567) (width 0.2) (layer "F.Cu") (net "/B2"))
 (segment (start 157.73 98) (end 157.73 99.0517) (width 0.2) (layer "F.Cu") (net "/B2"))
 (segment (start 137.7483 100.4375) (end 137.7483 101.5725) (width 0.2) (layer "F.Cu") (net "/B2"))
 (segment (start 157.73 99.0517) (end 139.1341 99.0517) (width 0.2) (layer "F.Cu") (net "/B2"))
 (segment (start 137.7483 101.5725) (end 138.0933 101.9175) (width 0.2) (layer "F.Cu") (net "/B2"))
 (segment (start 137.305 101.005) (end 137.305 102.0567) (width 0.2) (layer "F.Cu") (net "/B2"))
 (segment (start 138.0933 101.9175) (end 138.0933 102.0001) (width 0.2) (layer "F.Cu") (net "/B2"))
 (segment (start 139.845 101.005) (end 140.6717 101.005) (width 0.2) (layer "B.Cu") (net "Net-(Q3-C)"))
 (segment (start 119.8731 88.4731) (end 117.075 85.675) (width 0.2) (layer "B.Cu") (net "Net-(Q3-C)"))
 (segment (start 140.2243 107.8548) (end 130.1531 107.8548) (width 0.2) (layer "B.Cu") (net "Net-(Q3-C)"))
 (segment (start 140.7052 101.0385) (end 140.7052 107.3739) (width 0.2) (layer "B.Cu") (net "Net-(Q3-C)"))
 (segment (start 129.9683 107.67) (end 129.9683 106.979) (width 0.2) (layer "B.Cu") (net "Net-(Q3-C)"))
 (segment (start 130.1531 107.8548) (end 129.9683 107.67) (width 0.2) (layer "B.Cu") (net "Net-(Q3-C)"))
 (segment (start 140.7052 107.3739) (end 140.2243 107.8548) (width 0.2) (layer "B.Cu") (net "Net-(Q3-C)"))
 (segment (start 129.9683 106.979) (end 119.8731 96.8838) (width 0.2) (layer "B.Cu") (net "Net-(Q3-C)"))
 (segment (start 140.6717 101.005) (end 140.7052 101.0385) (width 0.2) (layer "B.Cu") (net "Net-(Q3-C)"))
 (segment (start 119.8731 96.8838) (end 119.8731 88.4731) (width 0.2) (layer "B.Cu") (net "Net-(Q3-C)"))
 (segment (start 132.0665 90.5065) (end 127.235 85.675) (width 0.2) (layer "B.Cu") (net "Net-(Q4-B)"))
 (segment (start 138.575 106.795) (end 138.575 104.5025) (width 0.2) (layer "B.Cu") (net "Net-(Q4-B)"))
 (segment (start 138.575 104.5025) (end 132.0665 97.994) (width 0.2) (layer "B.Cu") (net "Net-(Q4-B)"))
 (segment (start 132.0665 97.994) (end 132.0665 90.5065) (width 0.2) (layer "B.Cu") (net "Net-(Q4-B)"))
 (segment (start 155.23 116.5517) (end 174.23 116.5517) (width 0.2) (layer "F.Cu") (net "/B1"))
 (segment (start 175.23 114.5) (end 175.23 115.5517) (width 0.2) (layer "F.Cu") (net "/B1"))
 (segment (start 174.23 116.5517) (end 175.23 115.5517) (width 0.2) (layer "F.Cu") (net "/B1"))
 (segment (start 155.23 115.5) (end 155.23 116.5517) (width 0.2) (layer "F.Cu") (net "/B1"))
 (segment (start 146.5 102.86) (end 146.5 101.8083) (width 0.2) (layer "F.Cu") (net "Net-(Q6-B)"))
 (segment (start 130.5545 102.4662) (end 128.7975 100.7092) (width 0.2) (layer "F.Cu") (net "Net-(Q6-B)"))
 (segment (start 146.5 101.8083) (end 144.4063 101.8083) (width 0.2) (layer "F.Cu") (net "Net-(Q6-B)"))
 (segment (start 118.2408 100.7092) (end 117.075 101.875) (width 0.2) (layer "F.Cu") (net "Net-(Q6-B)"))
 (segment (start 143.7484 102.4662) (end 130.5545 102.4662) (width 0.2) (layer "F.Cu") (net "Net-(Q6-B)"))
 (segment (start 144.4063 101.8083) (end 143.7484 102.4662) (width 0.2) (layer "F.Cu") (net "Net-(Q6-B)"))
 (segment (start 128.7975 100.7092) (end 118.2408 100.7092) (width 0.2) (layer "F.Cu") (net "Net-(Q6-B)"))
 (segment (start 156.5 115.5) (end 156.5 114.4483) (width 0.2) (layer "F.Cu") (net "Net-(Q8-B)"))
 (segment (start 119.1 107.95) (end 117.075 105.925) (width 0.2) (layer "F.Cu") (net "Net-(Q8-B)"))
 (segment (start 127.7042 107.95) (end 119.1 107.95) (width 0.2) (layer "F.Cu") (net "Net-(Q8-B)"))
 (segment (start 156.5 114.4483) (end 134.2025 114.4483) (width 0.2) (layer "F.Cu") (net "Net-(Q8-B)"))
 (segment (start 134.2025 114.4483) (end 127.7042 107.95) (width 0.2) (layer "F.Cu") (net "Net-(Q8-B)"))
 (segment (start 157.3683 114.0466) (end 136.2793 114.0466) (width 0.2) (layer "F.Cu") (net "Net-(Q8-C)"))
 (segment (start 157.77 115.5) (end 157.77 114.4483) (width 0.2) (layer "F.Cu") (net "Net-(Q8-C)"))
 (segment (start 157.77 114.4483) (end 157.3683 114.0466) (width 0.2) (layer "F.Cu") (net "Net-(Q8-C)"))
 (segment (start 129.1525 103.7925) (end 127.235 101.875) (width 0.2) (layer "F.Cu") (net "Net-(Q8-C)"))
 (segment (start 136.2793 114.0466) (end 129.1525 106.9198) (width 0.2) (layer "F.Cu") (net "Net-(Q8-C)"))
 (segment (start 129.1525 106.9198) (end 129.1525 103.7925) (width 0.2) (layer "F.Cu") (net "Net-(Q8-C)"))
 (segment (start 132.8133 80.5233) (end 120.0233 80.5233) (width 0.2) (layer "F.Cu") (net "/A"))
 (segment (start 136.34 79.81) (end 135.2788 80.8712) (width 0.2) (layer "F.Cu") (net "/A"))
 (segment (start 120.0233 80.5233) (end 118.2463 82.3003) (width 0.2) (layer "F.Cu") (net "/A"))
 (segment (start 135.2788 80.8712) (end 133.1612 80.8712) (width 0.2) (layer "F.Cu") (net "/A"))
 (segment (start 118.2463 82.3003) (end 118.2463 87.7) (width 0.2) (layer "F.Cu") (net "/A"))
 (segment (start 133.1612 80.8712) (end 132.8133 80.5233) (width 0.2) (layer "F.Cu") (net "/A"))
 (via (at 118.2463 87.7) (size 0.6) (drill 0.3) (layers "F.Cu" "B.Cu") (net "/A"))
 (via (at 120.0233 80.5233) (size 0.6) (drill 0.3) (layers "F.Cu" "B.Cu") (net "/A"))
 (segment (start 117.075 77.575) (end 120.0233 80.5233) (width 0.2) (layer "B.Cu") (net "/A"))
 (segment (start 120.13 110.97) (end 127.235 118.075) (width 0.2) (layer "B.Cu") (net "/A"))
 (segment (start 118.2463 87.7) (end 118.2463 95.825) (width 0.2) (layer "B.Cu") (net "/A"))
 (segment (start 118.2463 95.825) (end 120.13 97.7087) (width 0.2) (layer "B.Cu") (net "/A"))
 (segment (start 120.13 97.7087) (end 120.13 110.97) (width 0.2) (layer "B.Cu") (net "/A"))
 (segment (start 127.235 89.725) (end 131.505 89.725) (width 0.2) (layer "F.Cu") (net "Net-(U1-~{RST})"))
 (segment (start 131.505 89.725) (end 138.88 82.35) (width 0.2) (layer "F.Cu") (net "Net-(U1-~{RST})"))
 (segment (start 127.235 93.775) (end 126.0984 92.6384) (width 0.2) (layer "F.Cu") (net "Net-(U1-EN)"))
 (segment (start 130.3225 88.3675) (end 136.34 82.35) (width 0.2) (layer "F.Cu") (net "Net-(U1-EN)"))
 (segment (start 126.0984 92.6384) (end 126.0984 89.2915) (width 0.2) (layer "F.Cu") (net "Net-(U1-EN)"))
 (segment (start 127.0224 88.3675) (end 130.3225 88.3675) (width 0.2) (layer "F.Cu") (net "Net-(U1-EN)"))
 (segment (start 126.0984 89.2915) (end 127.0224 88.3675) (width 0.2) (layer "F.Cu") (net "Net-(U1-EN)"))
 (segment (start 141.1069 107.5402) (end 141.1069 100.2583) (width 0.2) (layer "B.Cu") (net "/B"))
 (segment (start 140.3906 108.2565) (end 141.1069 107.5402) (width 0.2) (layer "B.Cu") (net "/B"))
 (segment (start 141.1069 100.2583) (end 140.15 99.3014) (width 0.2) (layer "B.Cu") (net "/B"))
 (segment (start 140.15 99.3014) (end 140.15 81.08) (width 0.2) (layer "B.Cu") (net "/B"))
 (segment (start 140.15 81.08) (end 138.88 79.81) (width 0.2) (layer "B.Cu") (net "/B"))
 (segment (start 129.5665 108.2565) (end 140.3906 108.2565) (width 0.2) (layer "B.Cu") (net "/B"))
 (segment (start 126.1302 107.0298) (end 127.235 105.925) (width 0.2) (layer "B.Cu") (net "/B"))
 (segment (start 126.1302 112.9202) (end 126.1302 107.0298) (width 0.2) (layer "B.Cu") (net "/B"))
 (segment (start 127.235 114.025) (end 126.1302 112.9202) (width 0.2) (layer "B.Cu") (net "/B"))
 (segment (start 127.235 105.925) (end 129.5665 108.2565) (width 0.2) (layer "B.Cu") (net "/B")))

